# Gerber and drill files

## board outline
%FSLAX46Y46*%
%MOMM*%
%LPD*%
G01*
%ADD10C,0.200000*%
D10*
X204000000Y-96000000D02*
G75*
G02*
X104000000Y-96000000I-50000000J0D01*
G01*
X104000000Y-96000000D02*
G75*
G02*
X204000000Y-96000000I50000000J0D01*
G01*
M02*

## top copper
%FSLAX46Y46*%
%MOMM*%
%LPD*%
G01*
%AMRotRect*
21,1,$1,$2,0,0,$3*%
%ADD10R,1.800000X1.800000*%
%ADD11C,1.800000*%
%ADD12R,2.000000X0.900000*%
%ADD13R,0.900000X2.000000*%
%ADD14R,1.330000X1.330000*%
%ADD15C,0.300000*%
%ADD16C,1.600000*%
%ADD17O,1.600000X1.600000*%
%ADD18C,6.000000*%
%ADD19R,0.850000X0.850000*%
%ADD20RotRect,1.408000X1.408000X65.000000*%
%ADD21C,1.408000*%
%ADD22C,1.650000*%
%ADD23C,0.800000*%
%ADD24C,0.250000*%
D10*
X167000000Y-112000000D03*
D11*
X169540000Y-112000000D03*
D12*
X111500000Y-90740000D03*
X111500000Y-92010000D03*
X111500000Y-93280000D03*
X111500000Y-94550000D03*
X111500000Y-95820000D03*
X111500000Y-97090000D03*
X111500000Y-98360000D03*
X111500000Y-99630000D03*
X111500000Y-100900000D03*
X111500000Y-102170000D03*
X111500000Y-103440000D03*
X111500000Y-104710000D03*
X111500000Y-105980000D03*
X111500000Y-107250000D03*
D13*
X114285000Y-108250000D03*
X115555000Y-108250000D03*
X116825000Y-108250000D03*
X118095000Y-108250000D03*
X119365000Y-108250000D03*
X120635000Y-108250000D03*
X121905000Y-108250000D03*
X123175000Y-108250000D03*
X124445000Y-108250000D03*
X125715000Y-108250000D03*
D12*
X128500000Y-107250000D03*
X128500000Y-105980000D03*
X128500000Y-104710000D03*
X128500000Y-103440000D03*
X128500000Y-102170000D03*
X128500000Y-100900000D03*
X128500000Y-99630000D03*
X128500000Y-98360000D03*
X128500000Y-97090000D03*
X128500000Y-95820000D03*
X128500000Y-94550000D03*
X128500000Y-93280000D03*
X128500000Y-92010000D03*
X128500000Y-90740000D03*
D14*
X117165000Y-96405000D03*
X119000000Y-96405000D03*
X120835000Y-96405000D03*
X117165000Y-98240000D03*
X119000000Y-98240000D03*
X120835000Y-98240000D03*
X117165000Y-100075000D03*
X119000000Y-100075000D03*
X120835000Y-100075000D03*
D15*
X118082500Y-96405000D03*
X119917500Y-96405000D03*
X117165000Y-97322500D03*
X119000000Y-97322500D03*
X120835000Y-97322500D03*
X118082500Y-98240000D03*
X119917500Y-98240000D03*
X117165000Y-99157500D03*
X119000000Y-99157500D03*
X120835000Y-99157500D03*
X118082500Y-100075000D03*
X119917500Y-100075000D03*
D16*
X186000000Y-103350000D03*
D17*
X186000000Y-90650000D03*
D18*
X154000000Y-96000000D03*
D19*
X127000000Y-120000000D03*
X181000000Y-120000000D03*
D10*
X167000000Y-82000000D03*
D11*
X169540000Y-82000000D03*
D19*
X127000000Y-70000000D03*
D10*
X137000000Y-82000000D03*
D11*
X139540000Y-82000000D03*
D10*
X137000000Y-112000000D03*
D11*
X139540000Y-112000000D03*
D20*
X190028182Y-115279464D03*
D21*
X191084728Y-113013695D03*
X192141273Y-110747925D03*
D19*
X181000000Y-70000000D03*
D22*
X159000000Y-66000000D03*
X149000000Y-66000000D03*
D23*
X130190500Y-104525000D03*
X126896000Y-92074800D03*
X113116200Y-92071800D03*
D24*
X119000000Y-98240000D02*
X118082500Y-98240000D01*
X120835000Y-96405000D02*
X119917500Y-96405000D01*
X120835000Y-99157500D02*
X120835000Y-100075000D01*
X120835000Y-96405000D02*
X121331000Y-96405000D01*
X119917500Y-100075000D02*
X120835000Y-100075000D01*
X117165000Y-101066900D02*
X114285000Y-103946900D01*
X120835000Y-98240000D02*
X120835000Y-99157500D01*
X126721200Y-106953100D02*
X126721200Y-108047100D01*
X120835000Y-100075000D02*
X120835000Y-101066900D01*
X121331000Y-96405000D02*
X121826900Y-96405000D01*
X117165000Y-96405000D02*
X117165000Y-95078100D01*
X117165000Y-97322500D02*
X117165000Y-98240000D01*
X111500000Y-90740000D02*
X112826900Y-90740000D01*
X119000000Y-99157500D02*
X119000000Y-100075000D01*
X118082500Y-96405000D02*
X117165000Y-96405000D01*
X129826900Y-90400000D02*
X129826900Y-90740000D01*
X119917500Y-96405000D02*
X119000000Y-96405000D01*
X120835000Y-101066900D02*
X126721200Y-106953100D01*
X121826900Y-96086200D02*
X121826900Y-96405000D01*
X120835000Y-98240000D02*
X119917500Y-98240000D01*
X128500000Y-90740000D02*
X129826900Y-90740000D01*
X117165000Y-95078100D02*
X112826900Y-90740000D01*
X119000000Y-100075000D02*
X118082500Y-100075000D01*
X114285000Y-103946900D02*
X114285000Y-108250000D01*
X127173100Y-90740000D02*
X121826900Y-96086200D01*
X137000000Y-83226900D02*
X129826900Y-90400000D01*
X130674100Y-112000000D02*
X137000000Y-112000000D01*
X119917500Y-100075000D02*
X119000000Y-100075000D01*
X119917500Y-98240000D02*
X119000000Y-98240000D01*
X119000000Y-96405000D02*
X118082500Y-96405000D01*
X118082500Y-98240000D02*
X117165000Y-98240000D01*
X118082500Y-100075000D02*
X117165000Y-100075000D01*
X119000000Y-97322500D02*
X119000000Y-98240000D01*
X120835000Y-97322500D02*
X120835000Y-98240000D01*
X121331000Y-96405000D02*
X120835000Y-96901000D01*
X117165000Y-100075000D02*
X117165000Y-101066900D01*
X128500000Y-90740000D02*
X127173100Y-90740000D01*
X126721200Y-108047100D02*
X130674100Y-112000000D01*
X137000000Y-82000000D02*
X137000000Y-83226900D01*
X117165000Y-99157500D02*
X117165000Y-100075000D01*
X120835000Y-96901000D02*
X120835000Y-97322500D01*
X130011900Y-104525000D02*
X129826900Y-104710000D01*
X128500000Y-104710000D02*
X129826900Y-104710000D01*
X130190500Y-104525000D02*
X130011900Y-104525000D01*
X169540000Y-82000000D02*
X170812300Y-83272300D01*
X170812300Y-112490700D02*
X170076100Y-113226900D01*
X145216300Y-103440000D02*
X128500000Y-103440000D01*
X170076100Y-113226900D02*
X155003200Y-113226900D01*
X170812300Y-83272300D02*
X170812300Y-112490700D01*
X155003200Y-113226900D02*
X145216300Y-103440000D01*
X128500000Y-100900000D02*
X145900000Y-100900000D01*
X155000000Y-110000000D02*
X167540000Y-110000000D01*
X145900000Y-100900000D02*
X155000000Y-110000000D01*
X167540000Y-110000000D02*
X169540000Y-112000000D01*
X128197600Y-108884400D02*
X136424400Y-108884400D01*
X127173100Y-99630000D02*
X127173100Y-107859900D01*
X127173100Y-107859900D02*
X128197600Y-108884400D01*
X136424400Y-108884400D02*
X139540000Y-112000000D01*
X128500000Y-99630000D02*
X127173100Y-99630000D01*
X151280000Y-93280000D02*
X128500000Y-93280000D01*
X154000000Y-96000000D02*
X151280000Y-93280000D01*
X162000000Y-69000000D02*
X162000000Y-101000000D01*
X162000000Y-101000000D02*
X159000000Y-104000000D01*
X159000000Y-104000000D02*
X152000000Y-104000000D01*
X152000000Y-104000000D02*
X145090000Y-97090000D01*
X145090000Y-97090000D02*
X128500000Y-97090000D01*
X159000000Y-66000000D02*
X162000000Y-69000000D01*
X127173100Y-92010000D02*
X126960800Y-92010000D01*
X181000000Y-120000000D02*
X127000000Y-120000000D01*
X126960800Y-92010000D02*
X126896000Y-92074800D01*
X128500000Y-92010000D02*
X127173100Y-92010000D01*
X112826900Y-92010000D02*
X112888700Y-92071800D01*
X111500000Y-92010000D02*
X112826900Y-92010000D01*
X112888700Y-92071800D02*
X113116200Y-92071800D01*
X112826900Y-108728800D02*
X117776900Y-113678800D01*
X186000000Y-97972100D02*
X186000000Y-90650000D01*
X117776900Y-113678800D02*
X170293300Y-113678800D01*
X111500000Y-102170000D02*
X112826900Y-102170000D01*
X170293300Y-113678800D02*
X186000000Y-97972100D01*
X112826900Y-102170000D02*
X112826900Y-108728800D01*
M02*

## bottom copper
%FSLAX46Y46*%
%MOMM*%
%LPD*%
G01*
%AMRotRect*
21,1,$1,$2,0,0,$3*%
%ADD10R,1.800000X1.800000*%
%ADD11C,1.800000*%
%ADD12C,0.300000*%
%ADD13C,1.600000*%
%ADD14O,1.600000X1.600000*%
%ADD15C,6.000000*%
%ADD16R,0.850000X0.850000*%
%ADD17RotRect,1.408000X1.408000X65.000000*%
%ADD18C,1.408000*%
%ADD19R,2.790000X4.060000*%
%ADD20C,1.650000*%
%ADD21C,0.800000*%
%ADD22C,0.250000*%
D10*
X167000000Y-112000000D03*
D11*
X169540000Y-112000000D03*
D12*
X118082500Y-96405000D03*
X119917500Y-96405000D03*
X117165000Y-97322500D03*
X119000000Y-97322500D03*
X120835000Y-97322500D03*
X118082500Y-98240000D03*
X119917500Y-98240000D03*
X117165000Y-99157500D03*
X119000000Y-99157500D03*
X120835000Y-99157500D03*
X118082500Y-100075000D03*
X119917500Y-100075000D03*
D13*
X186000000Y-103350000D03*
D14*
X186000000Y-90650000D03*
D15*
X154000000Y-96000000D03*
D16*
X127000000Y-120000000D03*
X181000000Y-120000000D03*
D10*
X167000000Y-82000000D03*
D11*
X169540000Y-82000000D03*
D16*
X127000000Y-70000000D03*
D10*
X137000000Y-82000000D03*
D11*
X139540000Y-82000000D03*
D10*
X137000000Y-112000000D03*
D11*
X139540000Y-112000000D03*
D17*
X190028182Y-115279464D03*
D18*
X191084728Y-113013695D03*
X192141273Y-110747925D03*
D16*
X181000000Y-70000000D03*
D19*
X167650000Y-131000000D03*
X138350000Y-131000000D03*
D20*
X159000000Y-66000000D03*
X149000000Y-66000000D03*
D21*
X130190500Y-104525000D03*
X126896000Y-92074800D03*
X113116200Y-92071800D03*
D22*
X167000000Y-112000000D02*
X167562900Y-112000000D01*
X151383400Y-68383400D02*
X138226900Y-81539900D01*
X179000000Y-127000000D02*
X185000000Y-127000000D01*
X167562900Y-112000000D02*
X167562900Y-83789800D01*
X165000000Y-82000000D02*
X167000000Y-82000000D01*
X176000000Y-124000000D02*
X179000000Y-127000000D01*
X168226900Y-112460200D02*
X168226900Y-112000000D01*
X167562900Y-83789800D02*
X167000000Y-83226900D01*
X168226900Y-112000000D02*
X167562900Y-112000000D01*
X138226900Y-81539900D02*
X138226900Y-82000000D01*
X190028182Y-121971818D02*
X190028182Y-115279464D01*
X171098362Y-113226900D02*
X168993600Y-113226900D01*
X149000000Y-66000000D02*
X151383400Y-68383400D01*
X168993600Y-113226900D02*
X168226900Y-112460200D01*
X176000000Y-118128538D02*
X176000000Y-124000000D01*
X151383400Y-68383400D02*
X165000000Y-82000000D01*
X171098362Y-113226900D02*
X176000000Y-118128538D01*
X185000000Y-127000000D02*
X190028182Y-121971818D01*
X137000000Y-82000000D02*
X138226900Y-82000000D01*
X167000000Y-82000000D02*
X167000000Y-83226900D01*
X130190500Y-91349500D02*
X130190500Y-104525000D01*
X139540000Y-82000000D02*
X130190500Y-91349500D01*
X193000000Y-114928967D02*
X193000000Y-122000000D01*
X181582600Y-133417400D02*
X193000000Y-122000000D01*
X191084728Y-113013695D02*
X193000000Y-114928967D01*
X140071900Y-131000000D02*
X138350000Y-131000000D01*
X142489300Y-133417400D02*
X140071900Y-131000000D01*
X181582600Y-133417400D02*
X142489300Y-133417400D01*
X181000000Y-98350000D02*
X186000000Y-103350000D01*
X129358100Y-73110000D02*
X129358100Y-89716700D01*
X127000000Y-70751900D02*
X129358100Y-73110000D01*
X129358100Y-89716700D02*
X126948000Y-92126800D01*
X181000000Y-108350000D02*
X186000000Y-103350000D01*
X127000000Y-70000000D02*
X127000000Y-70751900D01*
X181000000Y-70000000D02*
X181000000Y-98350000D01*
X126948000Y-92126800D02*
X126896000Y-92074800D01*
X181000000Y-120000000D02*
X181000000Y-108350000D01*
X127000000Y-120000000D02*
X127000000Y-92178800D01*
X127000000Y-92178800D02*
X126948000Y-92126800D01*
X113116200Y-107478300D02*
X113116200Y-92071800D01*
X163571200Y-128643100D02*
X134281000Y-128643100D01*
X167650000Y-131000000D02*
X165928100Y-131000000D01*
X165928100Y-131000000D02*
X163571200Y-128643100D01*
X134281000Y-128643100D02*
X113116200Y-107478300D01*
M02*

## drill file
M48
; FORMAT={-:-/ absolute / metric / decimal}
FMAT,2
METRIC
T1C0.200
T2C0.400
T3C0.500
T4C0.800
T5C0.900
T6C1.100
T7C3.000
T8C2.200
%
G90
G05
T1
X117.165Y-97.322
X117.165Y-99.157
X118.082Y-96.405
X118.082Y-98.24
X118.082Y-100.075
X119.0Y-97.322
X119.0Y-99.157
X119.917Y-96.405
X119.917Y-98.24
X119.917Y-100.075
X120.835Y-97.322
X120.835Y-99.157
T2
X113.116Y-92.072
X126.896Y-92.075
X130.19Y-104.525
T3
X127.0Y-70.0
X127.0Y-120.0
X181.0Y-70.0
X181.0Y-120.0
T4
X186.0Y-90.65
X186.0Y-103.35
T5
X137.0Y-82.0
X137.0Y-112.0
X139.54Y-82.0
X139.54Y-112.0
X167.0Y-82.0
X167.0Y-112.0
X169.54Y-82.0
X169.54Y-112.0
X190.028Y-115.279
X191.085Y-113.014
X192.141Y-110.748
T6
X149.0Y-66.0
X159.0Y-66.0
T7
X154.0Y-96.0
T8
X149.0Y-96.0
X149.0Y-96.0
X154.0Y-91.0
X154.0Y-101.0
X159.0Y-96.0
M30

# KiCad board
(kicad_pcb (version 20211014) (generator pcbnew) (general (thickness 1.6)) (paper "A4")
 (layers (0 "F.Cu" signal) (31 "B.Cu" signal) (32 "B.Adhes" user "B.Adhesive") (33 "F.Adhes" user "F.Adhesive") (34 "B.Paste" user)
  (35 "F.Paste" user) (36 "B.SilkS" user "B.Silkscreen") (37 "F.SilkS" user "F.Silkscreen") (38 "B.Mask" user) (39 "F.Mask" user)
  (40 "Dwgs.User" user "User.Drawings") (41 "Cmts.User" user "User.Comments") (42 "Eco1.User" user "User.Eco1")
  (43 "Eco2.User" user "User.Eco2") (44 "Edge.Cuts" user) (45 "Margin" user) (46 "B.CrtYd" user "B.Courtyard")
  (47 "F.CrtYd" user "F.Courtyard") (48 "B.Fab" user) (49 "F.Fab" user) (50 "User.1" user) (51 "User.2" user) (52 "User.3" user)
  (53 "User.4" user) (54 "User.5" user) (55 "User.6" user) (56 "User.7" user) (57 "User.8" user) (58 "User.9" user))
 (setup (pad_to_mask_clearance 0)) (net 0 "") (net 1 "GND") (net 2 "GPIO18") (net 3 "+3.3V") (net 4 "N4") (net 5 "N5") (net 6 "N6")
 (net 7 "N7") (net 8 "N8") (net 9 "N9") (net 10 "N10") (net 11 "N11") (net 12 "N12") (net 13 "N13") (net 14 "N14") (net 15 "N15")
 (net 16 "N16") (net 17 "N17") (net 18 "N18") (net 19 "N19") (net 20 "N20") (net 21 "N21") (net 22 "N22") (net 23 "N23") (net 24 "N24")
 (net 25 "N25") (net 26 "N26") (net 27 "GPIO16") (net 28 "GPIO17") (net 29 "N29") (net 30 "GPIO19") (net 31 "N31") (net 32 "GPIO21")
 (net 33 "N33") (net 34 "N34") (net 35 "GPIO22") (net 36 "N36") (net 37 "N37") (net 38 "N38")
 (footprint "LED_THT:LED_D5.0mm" (layer "F.Cu") (at 167 112)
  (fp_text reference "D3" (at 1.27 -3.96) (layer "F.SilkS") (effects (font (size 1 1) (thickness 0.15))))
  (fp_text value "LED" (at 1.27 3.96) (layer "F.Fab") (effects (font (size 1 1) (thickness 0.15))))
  (pad "1" thru_hole rect (at 0 0) (size 1.8 1.8) (drill 0.9) (layers *.Cu *.Mask) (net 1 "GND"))
  (pad "2" thru_hole circle (at 2.54 0) (size 1.8 1.8) (drill 0.9) (layers *.Cu *.Mask) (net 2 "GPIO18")))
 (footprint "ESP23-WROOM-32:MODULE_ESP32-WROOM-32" (layer "F.Cu") (at 120 96)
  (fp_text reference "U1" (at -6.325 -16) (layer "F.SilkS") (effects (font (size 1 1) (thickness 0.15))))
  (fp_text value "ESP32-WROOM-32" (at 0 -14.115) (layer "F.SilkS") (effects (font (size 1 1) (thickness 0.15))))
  (pad "1" smd rect locked (at -8.5 -5.26) (size 2 0.9) (layers "F.Cu" "F.Paste" "F.Mask") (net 1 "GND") (solder_mask_margin 0.102))
  (pad "2" smd rect locked (at -8.5 -3.99) (size 2 0.9) (layers "F.Cu" "F.Paste" "F.Mask") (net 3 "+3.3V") (solder_mask_margin 0.102))
  (pad "3" smd rect locked (at -8.5 -2.72) (size 2 0.9) (layers "F.Cu" "F.Paste" "F.Mask") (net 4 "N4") (solder_mask_margin 0.102))
  (pad "4" smd rect locked (at -8.5 -1.45) (size 2 0.9) (layers "F.Cu" "F.Paste" "F.Mask") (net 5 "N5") (solder_mask_margin 0.102))
  (pad "5" smd rect locked (at -8.5 -0.18) (size 2 0.9) (layers "F.Cu" "F.Paste" "F.Mask") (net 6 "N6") (solder_mask_margin 0.102))
  (pad "6" smd rect locked (at -8.5 1.09) (size 2 0.9) (layers "F.Cu" "F.Paste" "F.Mask") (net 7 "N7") (solder_mask_margin 0.102))
  (pad "7" smd rect locked (at -8.5 2.36) (size 2 0.9) (layers "F.Cu" "F.Paste" "F.Mask") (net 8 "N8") (solder_mask_margin 0.102))
  (pad "8" smd rect locked (at -8.5 3.63) (size 2 0.9) (layers "F.Cu" "F.Paste" "F.Mask") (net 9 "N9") (solder_mask_margin 0.102))
  (pad "9" smd rect locked (at -8.5 4.9) (size 2 0.9) (layers "F.Cu" "F.Paste" "F.Mask") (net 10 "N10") (solder_mask_margin 0.102))
  (pad "10" smd rect locked (at -8.5 6.17) (size 2 0.9) (layers "F.Cu" "F.Paste" "F.Mask") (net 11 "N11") (solder_mask_margin 0.102))
  (pad "11" smd rect locked (at -8.5 7.44) (size 2 0.9) (layers "F.Cu" "F.Paste" "F.Mask") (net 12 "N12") (solder_mask_margin 0.102))
  (pad "12" smd rect locked (at -8.5 8.71) (size 2 0.9) (layers "F.Cu" "F.Paste" "F.Mask") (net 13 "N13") (solder_mask_margin 0.102))
  (pad "13" smd rect locked (at -8.5 9.98) (size 2 0.9) (layers "F.Cu" "F.Paste" "F.Mask") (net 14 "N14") (solder_mask_margin 0.102))
  (pad "14" smd rect locked (at -8.5 11.25) (size 2 0.9) (layers "F.Cu" "F.Paste" "F.Mask") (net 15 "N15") (solder_mask_margin 0.102))
  (pad "15" smd rect locked (at -5.715 12.25) (size 0.9 2) (layers "F.Cu" "F.Paste" "F.Mask") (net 1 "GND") (solder_mask_margin 0.102))
  (pad "16" smd rect locked (at -4.445 12.25) (size 0.9 2) (layers "F.Cu" "F.Paste" "F.Mask") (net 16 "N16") (solder_mask_margin 0.102))
  (pad "17" smd rect locked (at -3.175 12.25) (size 0.9 2) (layers "F.Cu" "F.Paste" "F.Mask") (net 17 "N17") (solder_mask_margin 0.102))
  (pad "18" smd rect locked (at -1.905 12.25) (size 0.9 2) (layers "F.Cu" "F.Paste" "F.Mask") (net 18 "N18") (solder_mask_margin 0.102))
  (pad "19" smd rect locked (at -0.635 12.25) (size 0.9 2) (layers "F.Cu" "F.Paste" "F.Mask") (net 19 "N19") (solder_mask_margin 0.102))
  (pad "20" smd rect locked (at 0.635 12.25) (size 0.9 2) (layers "F.Cu" "F.Paste" "F.Mask") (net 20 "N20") (solder_mask_margin 0.102))
  (pad "21" smd rect locked (at 1.905 12.25) (size 0.9 2) (layers "F.Cu" "F.Paste" "F.Mask") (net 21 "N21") (solder_mask_margin 0.102))
  (pad "22" smd rect locked (at 3.175 12.25) (size 0.9 2) (layers "F.Cu" "F.Paste" "F.Mask") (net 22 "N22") (solder_mask_margin 0.102))
  (pad "23" smd rect locked (at 4.445 12.25) (size 0.9 2) (layers "F.Cu" "F.Paste" "F.Mask") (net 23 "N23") (solder_mask_margin 0.102))
  (pad "24" smd rect locked (at 5.715 12.25) (size 0.9 2) (layers "F.Cu" "F.Paste" "F.Mask") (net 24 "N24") (solder_mask_margin 0.102))
  (pad "25" smd rect locked (at 8.5 11.25) (size 2 0.9) (layers "F.Cu" "F.Paste" "F.Mask") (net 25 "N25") (solder_mask_margin 0.102))
  (pad "26" smd rect locked (at 8.5 9.98) (size 2 0.9) (layers "F.Cu" "F.Paste" "F.Mask") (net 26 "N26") (solder_mask_margin 0.102))
  (pad "27" smd rect locked (at 8.5 8.71) (size 2 0.9) (layers "F.Cu" "F.Paste" "F.Mask") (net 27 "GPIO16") (solder_mask_margin 0.102))
  (pad "28" smd rect locked (at 8.5 7.44) (size 2 0.9) (layers "F.Cu" "F.Paste" "F.Mask") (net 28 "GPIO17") (solder_mask_margin 0.102))
  (pad "29" smd rect locked (at 8.5 6.17) (size 2 0.9) (layers "F.Cu" "F.Paste" "F.Mask") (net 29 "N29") (solder_mask_margin 0.102))
  (pad "30" smd rect locked (at 8.5 4.9) (size 2 0.9) (layers "F.Cu" "F.Paste" "F.Mask") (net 2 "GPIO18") (solder_mask_margin 0.102))
  (pad "31" smd rect locked (at 8.5 3.63) (size 2 0.9) (layers "F.Cu" "F.Paste" "F.Mask") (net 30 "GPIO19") (solder_mask_margin 0.102))
  (pad "32" smd rect locked (at 8.5 2.36) (size 2 0.9) (layers "F.Cu" "F.Paste" "F.Mask") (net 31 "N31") (solder_mask_margin 0.102))
  (pad "33" smd rect locked (at 8.5 1.09) (size 2 0.9) (layers "F.Cu" "F.Paste" "F.Mask") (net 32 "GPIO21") (solder_mask_margin 0.102))
  (pad "34" smd rect locked (at 8.5 -0.18) (size 2 0.9) (layers "F.Cu" "F.Paste" "F.Mask") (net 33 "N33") (solder_mask_margin 0.102))
  (pad "35" smd rect locked (at 8.5 -1.45) (size 2 0.9) (layers "F.Cu" "F.Paste" "F.Mask") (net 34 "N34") (solder_mask_margin 0.102))
  (pad "36" smd rect locked (at 8.5 -2.72) (size 2 0.9) (layers "F.Cu" "F.Paste" "F.Mask") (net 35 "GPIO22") (solder_mask_margin 0.102))
  (pad "37" smd rect locked (at 8.5 -3.99) (size 2 0.9) (layers "F.Cu" "F.Paste" "F.Mask") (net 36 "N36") (solder_mask_margin 0.102))
  (pad "38" smd rect locked (at 8.5 -5.26) (size 2 0.9) (layers "F.Cu" "F.Paste" "F.Mask") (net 1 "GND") (solder_mask_margin 0.102))
  (pad "39_1" smd rect locked (at -2.835 0.405) (size 1.33 1.33) (layers "F.Cu" "F.Paste" "F.Mask") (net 1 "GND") (solder_mask_margin 0.102))
  (pad "39_2" smd rect locked (at -1 0.405) (size 1.33 1.33) (layers "F.Cu" "F.Paste" "F.Mask") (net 1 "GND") (solder_mask_margin 0.102))
  (pad "39_3" smd rect locked (at 0.835 0.405) (size 1.33 1.33) (layers "F.Cu" "F.Paste" "F.Mask") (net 1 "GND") (solder_mask_margin 0.102))
  (pad "39_4" smd rect locked (at -2.835 2.24) (size 1.33 1.33) (layers "F.Cu" "F.Paste" "F.Mask") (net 1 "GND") (solder_mask_margin 0.102))
  (pad "39_5" smd rect locked (at -1 2.24) (size 1.33 1.33) (layers "F.Cu" "F.Paste" "F.Mask") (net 1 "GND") (solder_mask_margin 0.102))
  (pad "39_6" smd rect locked (at 0.835 2.24) (size 1.33 1.33) (layers "F.Cu" "F.Paste" "F.Mask") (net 1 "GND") (solder_mask_margin 0.102))
  (pad "39_7" smd rect locked (at -2.835 4.075) (size 1.33 1.33) (layers "F.Cu" "F.Paste" "F.Mask") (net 1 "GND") (solder_mask_margin 0.102))
  (pad "39_8" smd rect locked (at -1 4.075) (size 1.33 1.33) (layers "F.Cu" "F.Paste" "F.Mask") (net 1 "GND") (solder_mask_margin 0.102))
  (pad "39_9" smd rect locked (at 0.835 4.075) (size 1.33 1.33) (layers "F.Cu" "F.Paste" "F.Mask") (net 1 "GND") (solder_mask_margin 0.102))
  (pad "39_10" thru_hole circle locked (at -1.9175 0.405) (size 0.3 0.3) (drill 0.2) (layers *.Cu *.Mask) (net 1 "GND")
   (solder_mask_margin 0.102))
  (pad "39_11" thru_hole circle locked (at -0.0825 0.405) (size 0.3 0.3) (drill 0.2) (layers *.Cu *.Mask) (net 1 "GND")
   (solder_mask_margin 0.102))
  (pad "39_12" thru_hole circle locked (at -2.835 1.3225) (size 0.3 0.3) (drill 0.2) (layers *.Cu *.Mask) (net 1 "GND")
   (solder_mask_margin 0.102))
  (pad "39_13" thru_hole circle locked (at -1 1.3225) (size 0.3 0.3) (drill 0.2) (layers *.Cu *.Mask) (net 1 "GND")
   (solder_mask_margin 0.102))
  (pad "39_14" thru_hole circle locked (at 0.835 1.3225) (size 0.3 0.3) (drill 0.2) (layers *.Cu *.Mask) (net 1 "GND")
   (solder_mask_margin 0.102))
  (pad "39_15" thru_hole circle locked (at -1.9175 2.24) (size 0.3 0.3) (drill 0.2) (layers *.Cu *.Mask) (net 1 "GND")
   (solder_mask_margin 0.102))
  (pad "39_16" thru_hole circle locked (at -0.0825 2.24) (size 0.3 0.3) (drill 0.2) (layers *.Cu *.Mask) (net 1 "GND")
   (solder_mask_margin 0.102))
  (pad "39_17" thru_hole circle locked (at -2.835 3.1575) (size 0.3 0.3) (drill 0.2) (layers *.Cu *.Mask) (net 1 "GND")
   (solder_mask_margin 0.102))
  (pad "39_18" thru_hole circle locked (at -1 3.1575) (size 0.3 0.3) (drill 0.2) (layers *.Cu *.Mask) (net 1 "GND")
   (solder_mask_margin 0.102))
  (pad "39_19" thru_hole circle locked (at 0.835 3.1575) (size 0.3 0.3) (drill 0.2) (layers *.Cu *.Mask) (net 1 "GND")
   (solder_mask_margin 0.102))
  (pad "39_20" thru_hole circle locked (at -1.9175 4.075) (size 0.3 0.3) (drill 0.2) (layers *.Cu *.Mask) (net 1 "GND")
   (solder_mask_margin 0.102))
  (pad "39_21" thru_hole circle locked (at -0.0825 4.075) (size 0.3 0.3) (drill 0.2) (layers *.Cu *.Mask) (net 1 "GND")
   (solder_mask_margin 0.102))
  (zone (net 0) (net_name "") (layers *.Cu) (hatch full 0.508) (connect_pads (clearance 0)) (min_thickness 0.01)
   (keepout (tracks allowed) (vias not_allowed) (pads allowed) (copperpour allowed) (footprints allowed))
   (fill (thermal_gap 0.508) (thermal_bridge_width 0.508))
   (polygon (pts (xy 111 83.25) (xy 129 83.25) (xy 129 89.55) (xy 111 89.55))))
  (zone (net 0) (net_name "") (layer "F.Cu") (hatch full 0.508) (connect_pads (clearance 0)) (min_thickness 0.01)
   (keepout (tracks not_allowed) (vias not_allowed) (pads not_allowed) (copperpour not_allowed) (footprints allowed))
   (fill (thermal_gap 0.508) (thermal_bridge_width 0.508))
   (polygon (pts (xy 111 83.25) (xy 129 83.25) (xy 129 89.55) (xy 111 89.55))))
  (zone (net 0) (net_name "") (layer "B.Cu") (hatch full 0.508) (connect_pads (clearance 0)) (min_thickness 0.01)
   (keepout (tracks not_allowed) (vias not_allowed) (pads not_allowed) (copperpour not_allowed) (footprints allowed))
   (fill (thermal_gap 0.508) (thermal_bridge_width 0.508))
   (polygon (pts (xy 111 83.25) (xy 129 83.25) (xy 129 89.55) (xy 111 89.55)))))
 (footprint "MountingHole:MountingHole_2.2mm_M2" (layer "F.Cu") (at 159 96)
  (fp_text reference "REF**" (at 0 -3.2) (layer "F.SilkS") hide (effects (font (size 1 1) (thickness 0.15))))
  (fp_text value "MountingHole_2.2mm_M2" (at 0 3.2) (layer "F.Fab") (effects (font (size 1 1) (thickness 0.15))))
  (pad "" np_thru_hole circle (at 0 0) (size 2.2 2.2) (drill 2.2) (layers *.Cu *.Mask)))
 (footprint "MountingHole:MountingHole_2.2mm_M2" (layer "F.Cu") (at 154 101)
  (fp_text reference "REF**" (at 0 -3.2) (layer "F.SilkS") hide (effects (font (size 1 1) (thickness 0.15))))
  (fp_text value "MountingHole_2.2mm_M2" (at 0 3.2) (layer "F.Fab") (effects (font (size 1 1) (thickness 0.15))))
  (pad "" np_thru_hole circle (at 0 0) (size 2.2 2.2) (drill 2.2) (layers *.Cu *.Mask)))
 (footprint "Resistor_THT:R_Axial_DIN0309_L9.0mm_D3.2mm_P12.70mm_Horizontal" (layer "F.Cu") (at 186 103.35 90)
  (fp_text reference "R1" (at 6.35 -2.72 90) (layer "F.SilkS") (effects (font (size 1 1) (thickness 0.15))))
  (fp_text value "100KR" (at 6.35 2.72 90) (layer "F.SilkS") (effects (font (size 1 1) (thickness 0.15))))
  (pad "1" thru_hole circle (at 0 0 90) (size 1.6 1.6) (drill 0.8) (layers *.Cu *.Mask) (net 36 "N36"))
  (pad "2" thru_hole oval (at 12.7 0 90) (size 1.6 1.6) (drill 0.8) (layers *.Cu *.Mask) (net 11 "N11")))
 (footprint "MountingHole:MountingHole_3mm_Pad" (layer "F.Cu") (at 154 96)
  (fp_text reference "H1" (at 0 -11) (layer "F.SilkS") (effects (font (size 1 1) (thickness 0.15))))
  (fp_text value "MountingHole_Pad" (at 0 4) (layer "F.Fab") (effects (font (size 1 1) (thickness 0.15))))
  (pad "1" thru_hole circle (at 0 0) (size 6 6) (drill 3) (layers *.Cu *.Mask) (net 35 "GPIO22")))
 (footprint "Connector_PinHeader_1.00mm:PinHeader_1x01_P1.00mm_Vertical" (layer "F.Cu") (at 127 120)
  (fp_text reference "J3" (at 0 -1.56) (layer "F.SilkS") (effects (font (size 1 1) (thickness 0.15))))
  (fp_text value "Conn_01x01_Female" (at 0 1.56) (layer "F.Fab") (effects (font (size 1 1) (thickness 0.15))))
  (pad "1" thru_hole rect (at 0 0) (size 0.85 0.85) (drill 0.5) (layers *.Cu *.Mask) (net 36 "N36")))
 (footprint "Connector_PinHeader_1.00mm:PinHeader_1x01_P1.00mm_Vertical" (layer "F.Cu") (at 181 120)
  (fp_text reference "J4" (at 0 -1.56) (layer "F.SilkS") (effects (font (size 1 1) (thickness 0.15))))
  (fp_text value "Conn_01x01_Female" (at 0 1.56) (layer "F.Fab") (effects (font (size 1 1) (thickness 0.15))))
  (pad "1" thru_hole rect (at 0 0) (size 0.85 0.85) (drill 0.5) (layers *.Cu *.Mask) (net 36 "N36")))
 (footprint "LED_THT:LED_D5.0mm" (layer "F.Cu") (at 167 82)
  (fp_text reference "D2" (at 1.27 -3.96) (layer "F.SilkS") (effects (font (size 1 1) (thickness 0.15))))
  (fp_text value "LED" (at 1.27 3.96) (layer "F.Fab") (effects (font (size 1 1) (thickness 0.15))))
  (pad "1" thru_hole rect (at 0 0) (size 1.8 1.8) (drill 0.9) (layers *.Cu *.Mask) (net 1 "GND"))
  (pad "2" thru_hole circle (at 2.54 0) (size 1.8 1.8) (drill 0.9) (layers *.Cu *.Mask) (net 28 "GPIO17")))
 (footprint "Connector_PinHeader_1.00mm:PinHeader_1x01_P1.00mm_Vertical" (layer "F.Cu") (at 127 70)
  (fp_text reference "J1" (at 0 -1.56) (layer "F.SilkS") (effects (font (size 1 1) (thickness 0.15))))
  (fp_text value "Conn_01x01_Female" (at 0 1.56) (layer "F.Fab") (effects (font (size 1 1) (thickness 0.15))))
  (pad "1" thru_hole rect (at 0 0) (size 0.85 0.85) (drill 0.5) (layers *.Cu *.Mask) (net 36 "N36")))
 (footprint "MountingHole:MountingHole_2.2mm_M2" (layer "F.Cu") (at 154 91)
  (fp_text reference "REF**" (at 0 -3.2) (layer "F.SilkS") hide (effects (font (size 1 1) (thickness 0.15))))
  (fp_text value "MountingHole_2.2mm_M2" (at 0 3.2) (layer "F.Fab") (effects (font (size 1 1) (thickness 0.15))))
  (pad "" np_thru_hole circle (at 0 0) (size 2.2 2.2) (drill 2.2) (layers *.Cu *.Mask)))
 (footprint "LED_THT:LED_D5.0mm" (layer "F.Cu") (at 137 82)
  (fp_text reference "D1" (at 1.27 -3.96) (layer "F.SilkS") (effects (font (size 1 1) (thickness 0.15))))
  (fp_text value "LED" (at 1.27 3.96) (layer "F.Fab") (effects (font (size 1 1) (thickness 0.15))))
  (pad "1" thru_hole rect (at 0 0) (size 1.8 1.8) (drill 0.9) (layers *.Cu *.Mask) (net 1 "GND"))
  (pad "2" thru_hole circle (at 2.54 0) (size 1.8 1.8) (drill 0.9) (layers *.Cu *.Mask) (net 27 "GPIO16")))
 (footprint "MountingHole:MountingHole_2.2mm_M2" (layer "F.Cu") (at 149 96)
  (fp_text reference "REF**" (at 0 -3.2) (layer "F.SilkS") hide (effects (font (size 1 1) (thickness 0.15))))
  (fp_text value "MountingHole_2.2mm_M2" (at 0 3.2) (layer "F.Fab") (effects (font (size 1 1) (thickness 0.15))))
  (pad "" np_thru_hole circle (at 0 0) (size 2.2 2.2) (drill 2.2) (layers *.Cu *.Mask))
  (pad "" np_thru_hole circle (at 0 0) (size 2.2 2.2) (drill 2.2) (layers *.Cu *.Mask)))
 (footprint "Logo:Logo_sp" (layer "F.Cu") (at 153 132)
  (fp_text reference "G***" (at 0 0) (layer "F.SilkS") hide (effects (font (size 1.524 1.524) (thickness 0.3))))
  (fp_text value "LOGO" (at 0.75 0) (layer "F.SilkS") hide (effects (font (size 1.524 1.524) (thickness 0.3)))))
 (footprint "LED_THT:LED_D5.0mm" (layer "F.Cu") (at 137 112)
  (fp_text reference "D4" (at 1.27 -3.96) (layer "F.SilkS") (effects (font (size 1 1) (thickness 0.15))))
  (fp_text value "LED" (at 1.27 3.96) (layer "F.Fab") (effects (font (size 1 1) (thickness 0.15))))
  (pad "1" thru_hole rect (at 0 0) (size 1.8 1.8) (drill 0.9) (layers *.Cu *.Mask) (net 1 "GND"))
  (pad "2" thru_hole circle (at 2.54 0) (size 1.8 1.8) (drill 0.9) (layers *.Cu *.Mask) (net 30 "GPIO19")))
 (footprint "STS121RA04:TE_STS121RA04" (layer "F.Cu") (at 190.028182 115.279464 65)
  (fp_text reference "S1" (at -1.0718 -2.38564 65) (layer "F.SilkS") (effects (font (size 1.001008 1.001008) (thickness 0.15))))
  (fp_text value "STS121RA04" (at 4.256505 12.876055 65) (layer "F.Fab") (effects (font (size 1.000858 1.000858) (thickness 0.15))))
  (pad "1" thru_hole rect locked (at 0 0 65) (size 1.408 1.408) (drill 0.9) (layers *.Cu *.Mask) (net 1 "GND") (solder_mask_margin 0.102))
  (pad "2" thru_hole circle locked (at 2.5 0 65) (size 1.408 1.408) (drill 0.9) (layers *.Cu *.Mask) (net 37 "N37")
   (solder_mask_margin 0.102))
  (pad "3" thru_hole circle locked (at 5 0 65) (size 1.408 1.408) (drill 0.9) (layers *.Cu *.Mask) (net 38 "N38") (solder_mask_margin 0.102)))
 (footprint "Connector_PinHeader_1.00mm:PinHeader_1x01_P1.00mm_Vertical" (layer "F.Cu") (at 181 70)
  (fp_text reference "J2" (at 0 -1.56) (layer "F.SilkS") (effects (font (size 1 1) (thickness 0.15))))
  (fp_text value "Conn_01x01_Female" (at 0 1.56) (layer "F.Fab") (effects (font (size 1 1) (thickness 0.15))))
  (pad "1" thru_hole rect (at 0 0) (size 0.85 0.85) (drill 0.5) (layers *.Cu *.Mask) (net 36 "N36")))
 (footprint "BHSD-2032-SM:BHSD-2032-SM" (layer "B.Cu") (at 153 131 180)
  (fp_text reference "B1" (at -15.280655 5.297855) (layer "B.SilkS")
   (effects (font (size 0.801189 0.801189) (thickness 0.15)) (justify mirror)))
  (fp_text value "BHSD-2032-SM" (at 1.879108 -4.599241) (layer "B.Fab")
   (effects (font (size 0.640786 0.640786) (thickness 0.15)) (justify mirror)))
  (pad "+" smd rect locked (at -14.65 0 180) (size 2.79 4.06) (layers "B.Cu" "B.Paste" "B.Mask") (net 3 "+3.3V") (solder_mask_margin 0.102))
  (pad "-" smd rect locked (at 14.65 0 180) (size 2.79 4.06) (layers "B.Cu" "B.Paste" "B.Mask") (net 37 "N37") (solder_mask_margin 0.102)))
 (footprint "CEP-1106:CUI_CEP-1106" (layer "B.Cu") (at 154 66 180)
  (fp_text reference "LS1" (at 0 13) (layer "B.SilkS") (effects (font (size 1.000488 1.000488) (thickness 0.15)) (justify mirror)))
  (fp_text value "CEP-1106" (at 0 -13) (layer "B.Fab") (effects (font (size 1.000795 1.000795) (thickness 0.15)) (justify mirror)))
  (pad "1" thru_hole circle locked (at -5 0 180) (size 1.65 1.65) (drill 1.1) (layers *.Cu *.Mask) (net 32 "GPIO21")
   (solder_mask_margin 0.102))
  (pad "2" thru_hole circle locked (at 5 0 180) (size 1.65 1.65) (drill 1.1) (layers *.Cu *.Mask) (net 1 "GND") (solder_mask_margin 0.102)))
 (gr_circle (center 154 96) (end 204 96) (layer "Edge.Cuts") (width 0.2) (fill none))
 (segment (start 119 98.24) (end 118.0825 98.24) (width 0.25) (layer "F.Cu") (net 1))
 (segment (start 120.835 96.405) (end 119.9175 96.405) (width 0.25) (layer "F.Cu") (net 1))
 (segment (start 120.835 99.1575) (end 120.835 100.075) (width 0.25) (layer "F.Cu") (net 1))
 (segment (start 120.835 96.405) (end 121.331 96.405) (width 0.25) (layer "F.Cu") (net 1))
 (segment (start 119.9175 100.075) (end 120.835 100.075) (width 0.25) (layer "F.Cu") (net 1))
 (segment (start 117.165 101.0669) (end 114.285 103.9469) (width 0.25) (layer "F.Cu") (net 1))
 (segment (start 120.835 98.24) (end 120.835 99.1575) (width 0.25) (layer "F.Cu") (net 1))
 (segment (start 126.7212 106.9531) (end 126.7212 108.0471) (width 0.25) (layer "F.Cu") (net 1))
 (segment (start 120.835 100.075) (end 120.835 101.0669) (width 0.25) (layer "F.Cu") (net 1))
 (segment (start 121.331 96.405) (end 121.8269 96.405) (width 0.25) (layer "F.Cu") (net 1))
 (segment (start 117.165 96.405) (end 117.165 95.0781) (width 0.25) (layer "F.Cu") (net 1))
 (segment (start 117.165 97.3225) (end 117.165 98.24) (width 0.25) (layer "F.Cu") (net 1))
 (segment (start 111.5 90.74) (end 112.8269 90.74) (width 0.25) (layer "F.Cu") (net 1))
 (segment (start 119 99.1575) (end 119 100.075) (width 0.25) (layer "F.Cu") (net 1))
 (segment (start 118.0825 96.405) (end 117.165 96.405) (width 0.25) (layer "F.Cu") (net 1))
 (segment (start 129.8269 90.4) (end 129.8269 90.74) (width 0.25) (layer "F.Cu") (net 1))
 (segment (start 119.9175 96.405) (end 119 96.405) (width 0.25) (layer "F.Cu") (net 1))
 (segment (start 120.835 101.0669) (end 126.7212 106.9531) (width 0.25) (layer "F.Cu") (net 1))
 (segment (start 121.8269 96.0862) (end 121.8269 96.405) (width 0.25) (layer "F.Cu") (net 1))
 (segment (start 120.835 98.24) (end 119.9175 98.24) (width 0.25) (layer "F.Cu") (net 1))
 (segment (start 128.5 90.74) (end 129.8269 90.74) (width 0.25) (layer "F.Cu") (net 1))
 (segment (start 117.165 95.0781) (end 112.8269 90.74) (width 0.25) (layer "F.Cu") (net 1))
 (segment (start 119 100.075) (end 118.0825 100.075) (width 0.25) (layer "F.Cu") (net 1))
 (segment (start 114.285 103.9469) (end 114.285 108.25) (width 0.25) (layer "F.Cu") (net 1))
 (segment (start 127.1731 90.74) (end 121.8269 96.0862) (width 0.25) (layer "F.Cu") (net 1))
 (segment (start 137 83.2269) (end 129.8269 90.4) (width 0.25) (layer "F.Cu") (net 1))
 (segment (start 130.6741 112) (end 137 112) (width 0.25) (layer "F.Cu") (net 1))
 (segment (start 119.9175 100.075) (end 119 100.075) (width 0.25) (layer "F.Cu") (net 1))
 (segment (start 119.9175 98.24) (end 119 98.24) (width 0.25) (layer "F.Cu") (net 1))
 (segment (start 119 96.405) (end 118.0825 96.405) (width 0.25) (layer "F.Cu") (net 1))
 (segment (start 118.0825 98.24) (end 117.165 98.24) (width 0.25) (layer "F.Cu") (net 1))
 (segment (start 118.0825 100.075) (end 117.165 100.075) (width 0.25) (layer "F.Cu") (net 1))
 (segment (start 119 97.3225) (end 119 98.24) (width 0.25) (layer "F.Cu") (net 1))
 (segment (start 120.835 97.3225) (end 120.835 98.24) (width 0.25) (layer "F.Cu") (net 1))
 (segment (start 121.331 96.405) (end 120.835 96.901) (width 0.25) (layer "F.Cu") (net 1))
 (segment (start 117.165 100.075) (end 117.165 101.0669) (width 0.25) (layer "F.Cu") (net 1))
 (segment (start 128.5 90.74) (end 127.1731 90.74) (width 0.25) (layer "F.Cu") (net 1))
 (segment (start 126.7212 108.0471) (end 130.6741 112) (width 0.25) (layer "F.Cu") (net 1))
 (segment (start 137 82) (end 137 83.2269) (width 0.25) (layer "F.Cu") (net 1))
 (segment (start 117.165 99.1575) (end 117.165 100.075) (width 0.25) (layer "F.Cu") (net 1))
 (segment (start 120.835 96.901) (end 120.835 97.3225) (width 0.25) (layer "F.Cu") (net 1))
 (segment (start 167 112) (end 167.5629 112) (width 0.25) (layer "B.Cu") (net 1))
 (segment (start 151.3834 68.3834) (end 138.2269 81.5399) (width 0.25) (layer "B.Cu") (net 1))
 (segment (start 179 127) (end 185 127) (width 0.25) (layer "B.Cu") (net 1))
 (segment (start 167.5629 112) (end 167.5629 83.7898) (width 0.25) (layer "B.Cu") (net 1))
 (segment (start 165 82) (end 167 82) (width 0.25) (layer "B.Cu") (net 1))
 (segment (start 176 124) (end 179 127) (width 0.25) (layer "B.Cu") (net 1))
 (segment (start 168.2269 112.4602) (end 168.2269 112) (width 0.25) (layer "B.Cu") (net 1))
 (segment (start 167.5629 83.7898) (end 167 83.2269) (width 0.25) (layer "B.Cu") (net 1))
 (segment (start 168.2269 112) (end 167.5629 112) (width 0.25) (layer "B.Cu") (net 1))
 (segment (start 138.2269 81.5399) (end 138.2269 82) (width 0.25) (layer "B.Cu") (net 1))
 (segment (start 190.028182 121.971818) (end 190.028182 115.279464) (width 0.25) (layer "B.Cu") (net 1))
 (segment (start 171.098362 113.2269) (end 168.9936 113.2269) (width 0.25) (layer "B.Cu") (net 1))
 (segment (start 149 66) (end 151.3834 68.3834) (width 0.25) (layer "B.Cu") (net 1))
 (segment (start 168.9936 113.2269) (end 168.2269 112.4602) (width 0.25) (layer "B.Cu") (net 1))
 (segment (start 176 118.128538) (end 176 124) (width 0.25) (layer "B.Cu") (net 1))
 (segment (start 151.3834 68.3834) (end 165 82) (width 0.25) (layer "B.Cu") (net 1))
 (segment (start 171.098362 113.2269) (end 176 118.128538) (width 0.25) (layer "B.Cu") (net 1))
 (segment (start 185 127) (end 190.028182 121.971818) (width 0.25) (layer "B.Cu") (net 1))
 (segment (start 137 82) (end 138.2269 82) (width 0.25) (layer "B.Cu") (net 1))
 (segment (start 167 82) (end 167 83.2269) (width 0.25) (layer "B.Cu") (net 1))
 (segment (start 130.0119 104.525) (end 129.8269 104.71) (width 0.25) (layer "F.Cu") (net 27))
 (segment (start 128.5 104.71) (end 129.8269 104.71) (width 0.25) (layer "F.Cu") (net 27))
 (segment (start 130.1905 104.525) (end 130.0119 104.525) (width 0.25) (layer "F.Cu") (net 27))
 (via (at 130.1905 104.525) (size 0.8) (drill 0.4) (layers "F.Cu" "B.Cu") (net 27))
 (segment (start 130.1905 91.3495) (end 130.1905 104.525) (width 0.25) (layer "B.Cu") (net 27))
 (segment (start 139.54 82) (end 130.1905 91.3495) (width 0.25) (layer "B.Cu") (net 27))
 (segment (start 169.54 82) (end 170.8123 83.2723) (width 0.25) (layer "F.Cu") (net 28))
 (segment (start 170.8123 112.4907) (end 170.0761 113.2269) (width 0.25) (layer "F.Cu") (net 28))
 (segment (start 145.2163 103.44) (end 128.5 103.44) (width 0.25) (layer "F.Cu") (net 28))
 (segment (start 170.0761 113.2269) (end 155.0032 113.2269) (width 0.25) (layer "F.Cu") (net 28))
 (segment (start 170.8123 83.2723) (end 170.8123 112.4907) (width 0.25) (layer "F.Cu") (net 28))
 (segment (start 155.0032 113.2269) (end 145.2163 103.44) (width 0.25) (layer "F.Cu") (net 28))
 (segment (start 128.5 100.9) (end 145.9 100.9) (width 0.25) (layer "F.Cu") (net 2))
 (segment (start 155 110) (end 167.54 110) (width 0.25) (layer "F.Cu") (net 2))
 (segment (start 145.9 100.9) (end 155 110) (width 0.25) (layer "F.Cu") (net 2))
 (segment (start 167.54 110) (end 169.54 112) (width 0.25) (layer "F.Cu") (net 2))
 (segment (start 128.1976 108.8844) (end 136.4244 108.8844) (width 0.25) (layer "F.Cu") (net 30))
 (segment (start 127.1731 99.63) (end 127.1731 107.8599) (width 0.25) (layer "F.Cu") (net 30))
 (segment (start 127.1731 107.8599) (end 128.1976 108.8844) (width 0.25) (layer "F.Cu") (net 30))
 (segment (start 136.4244 108.8844) (end 139.54 112) (width 0.25) (layer "F.Cu") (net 30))
 (segment (start 128.5 99.63) (end 127.1731 99.63) (width 0.25) (layer "F.Cu") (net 30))
 (segment (start 151.28 93.28) (end 128.5 93.28) (width 0.25) (layer "F.Cu") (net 35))
 (segment (start 154 96) (end 151.28 93.28) (width 0.25) (layer "F.Cu") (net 35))
 (segment (start 162 69) (end 162 101) (width 0.25) (layer "F.Cu") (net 32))
 (segment (start 162 101) (end 159 104) (width 0.25) (layer "F.Cu") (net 32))
 (segment (start 159 104) (end 152 104) (width 0.25) (layer "F.Cu") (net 32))
 (segment (start 152 104) (end 145.09 97.09) (width 0.25) (layer "F.Cu") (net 32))
 (segment (start 145.09 97.09) (end 128.5 97.09) (width 0.25) (layer "F.Cu") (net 32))
 (segment (start 159 66) (end 162 69) (width 0.25) (layer "F.Cu") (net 32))
 (segment (start 193 114.928967) (end 193 122) (width 0.25) (layer "B.Cu") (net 37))
 (segment (start 181.5826 133.4174) (end 193 122) (width 0.25) (layer "B.Cu") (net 37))
 (segment (start 191.084728 113.013695) (end 193 114.928967) (width 0.25) (layer "B.Cu") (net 37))
 (segment (start 140.0719 131) (end 138.35 131) (width 0.25) (layer "B.Cu") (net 37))
 (segment (start 142.4893 133.4174) (end 140.0719 131) (width 0.25) (layer "B.Cu") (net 37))
 (segment (start 181.5826 133.4174) (end 142.4893 133.4174) (width 0.25) (layer "B.Cu") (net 37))
 (segment (start 127.1731 92.01) (end 126.9608 92.01) (width 0.25) (layer "F.Cu") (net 36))
 (segment (start 181 120) (end 127 120) (width 0.25) (layer "F.Cu") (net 36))
 (segment (start 126.9608 92.01) (end 126.896 92.0748) (width 0.25) (layer "F.Cu") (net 36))
 (segment (start 128.5 92.01) (end 127.1731 92.01) (width 0.25) (layer "F.Cu") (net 36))
 (via (at 126.896 92.0748) (size 0.8) (drill 0.4) (layers "F.Cu" "B.Cu") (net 36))
 (segment (start 181 98.35) (end 186 103.35) (width 0.25) (layer "B.Cu") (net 36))
 (segment (start 129.3581 73.11) (end 129.3581 89.7167) (width 0.25) (layer "B.Cu") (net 36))
 (segment (start 127 70.7519) (end 129.3581 73.11) (width 0.25) (layer "B.Cu") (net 36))
 (segment (start 129.3581 89.7167) (end 126.948 92.1268) (width 0.25) (layer "B.Cu") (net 36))
 (segment (start 181 108.35) (end 186 103.35) (width 0.25) (layer "B.Cu") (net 36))
 (segment (start 127 70) (end 127 70.7519) (width 0.25) (layer "B.Cu") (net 36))
 (segment (start 181 70) (end 181 98.35) (width 0.25) (layer "B.Cu") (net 36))
 (segment (start 126.948 92.1268) (end 126.896 92.0748) (width 0.25) (layer "B.Cu") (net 36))
 (segment (start 181 120) (end 181 108.35) (width 0.25) (layer "B.Cu") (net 36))
 (segment (start 127 120) (end 127 92.1788) (width 0.25) (layer "B.Cu") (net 36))
 (segment (start 127 92.1788) (end 126.948 92.1268) (width 0.25) (layer "B.Cu") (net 36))
 (segment (start 112.8269 92.01) (end 112.8887 92.0718) (width 0.25) (layer "F.Cu") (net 3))
 (segment (start 111.5 92.01) (end 112.8269 92.01) (width 0.25) (layer "F.Cu") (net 3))
 (segment (start 112.8887 92.0718) (end 113.1162 92.0718) (width 0.25) (layer "F.Cu") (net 3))
 (via (at 113.1162 92.0718) (size 0.8) (drill 0.4) (layers "F.Cu" "B.Cu") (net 3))
 (segment (start 113.1162 107.4783) (end 113.1162 92.0718) (width 0.25) (layer "B.Cu") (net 3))
 (segment (start 163.5712 128.6431) (end 134.281 128.6431) (width 0.25) (layer "B.Cu") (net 3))
 (segment (start 167.65 131) (end 165.9281 131) (width 0.25) (layer "B.Cu") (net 3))
 (segment (start 165.9281 131) (end 163.5712 128.6431) (width 0.25) (layer "B.Cu") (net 3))
 (segment (start 134.281 128.6431) (end 113.1162 107.4783) (width 0.25) (layer "B.Cu") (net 3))
 (segment (start 112.8269 108.7288) (end 117.7769 113.6788) (width 0.25) (layer "F.Cu") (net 11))
 (segment (start 186 97.9721) (end 186 90.65) (width 0.25) (layer "F.Cu") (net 11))
 (segment (start 117.7769 113.6788) (end 170.2933 113.6788) (width 0.25) (layer "F.Cu") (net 11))
 (segment (start 111.5 102.17) (end 112.8269 102.17) (width 0.25) (layer "F.Cu") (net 11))
 (segment (start 170.2933 113.6788) (end 186 97.9721) (width 0.25) (layer "F.Cu") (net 11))
 (segment (start 112.8269 102.17) (end 112.8269 108.7288) (width 0.25) (layer "F.Cu") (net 11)))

